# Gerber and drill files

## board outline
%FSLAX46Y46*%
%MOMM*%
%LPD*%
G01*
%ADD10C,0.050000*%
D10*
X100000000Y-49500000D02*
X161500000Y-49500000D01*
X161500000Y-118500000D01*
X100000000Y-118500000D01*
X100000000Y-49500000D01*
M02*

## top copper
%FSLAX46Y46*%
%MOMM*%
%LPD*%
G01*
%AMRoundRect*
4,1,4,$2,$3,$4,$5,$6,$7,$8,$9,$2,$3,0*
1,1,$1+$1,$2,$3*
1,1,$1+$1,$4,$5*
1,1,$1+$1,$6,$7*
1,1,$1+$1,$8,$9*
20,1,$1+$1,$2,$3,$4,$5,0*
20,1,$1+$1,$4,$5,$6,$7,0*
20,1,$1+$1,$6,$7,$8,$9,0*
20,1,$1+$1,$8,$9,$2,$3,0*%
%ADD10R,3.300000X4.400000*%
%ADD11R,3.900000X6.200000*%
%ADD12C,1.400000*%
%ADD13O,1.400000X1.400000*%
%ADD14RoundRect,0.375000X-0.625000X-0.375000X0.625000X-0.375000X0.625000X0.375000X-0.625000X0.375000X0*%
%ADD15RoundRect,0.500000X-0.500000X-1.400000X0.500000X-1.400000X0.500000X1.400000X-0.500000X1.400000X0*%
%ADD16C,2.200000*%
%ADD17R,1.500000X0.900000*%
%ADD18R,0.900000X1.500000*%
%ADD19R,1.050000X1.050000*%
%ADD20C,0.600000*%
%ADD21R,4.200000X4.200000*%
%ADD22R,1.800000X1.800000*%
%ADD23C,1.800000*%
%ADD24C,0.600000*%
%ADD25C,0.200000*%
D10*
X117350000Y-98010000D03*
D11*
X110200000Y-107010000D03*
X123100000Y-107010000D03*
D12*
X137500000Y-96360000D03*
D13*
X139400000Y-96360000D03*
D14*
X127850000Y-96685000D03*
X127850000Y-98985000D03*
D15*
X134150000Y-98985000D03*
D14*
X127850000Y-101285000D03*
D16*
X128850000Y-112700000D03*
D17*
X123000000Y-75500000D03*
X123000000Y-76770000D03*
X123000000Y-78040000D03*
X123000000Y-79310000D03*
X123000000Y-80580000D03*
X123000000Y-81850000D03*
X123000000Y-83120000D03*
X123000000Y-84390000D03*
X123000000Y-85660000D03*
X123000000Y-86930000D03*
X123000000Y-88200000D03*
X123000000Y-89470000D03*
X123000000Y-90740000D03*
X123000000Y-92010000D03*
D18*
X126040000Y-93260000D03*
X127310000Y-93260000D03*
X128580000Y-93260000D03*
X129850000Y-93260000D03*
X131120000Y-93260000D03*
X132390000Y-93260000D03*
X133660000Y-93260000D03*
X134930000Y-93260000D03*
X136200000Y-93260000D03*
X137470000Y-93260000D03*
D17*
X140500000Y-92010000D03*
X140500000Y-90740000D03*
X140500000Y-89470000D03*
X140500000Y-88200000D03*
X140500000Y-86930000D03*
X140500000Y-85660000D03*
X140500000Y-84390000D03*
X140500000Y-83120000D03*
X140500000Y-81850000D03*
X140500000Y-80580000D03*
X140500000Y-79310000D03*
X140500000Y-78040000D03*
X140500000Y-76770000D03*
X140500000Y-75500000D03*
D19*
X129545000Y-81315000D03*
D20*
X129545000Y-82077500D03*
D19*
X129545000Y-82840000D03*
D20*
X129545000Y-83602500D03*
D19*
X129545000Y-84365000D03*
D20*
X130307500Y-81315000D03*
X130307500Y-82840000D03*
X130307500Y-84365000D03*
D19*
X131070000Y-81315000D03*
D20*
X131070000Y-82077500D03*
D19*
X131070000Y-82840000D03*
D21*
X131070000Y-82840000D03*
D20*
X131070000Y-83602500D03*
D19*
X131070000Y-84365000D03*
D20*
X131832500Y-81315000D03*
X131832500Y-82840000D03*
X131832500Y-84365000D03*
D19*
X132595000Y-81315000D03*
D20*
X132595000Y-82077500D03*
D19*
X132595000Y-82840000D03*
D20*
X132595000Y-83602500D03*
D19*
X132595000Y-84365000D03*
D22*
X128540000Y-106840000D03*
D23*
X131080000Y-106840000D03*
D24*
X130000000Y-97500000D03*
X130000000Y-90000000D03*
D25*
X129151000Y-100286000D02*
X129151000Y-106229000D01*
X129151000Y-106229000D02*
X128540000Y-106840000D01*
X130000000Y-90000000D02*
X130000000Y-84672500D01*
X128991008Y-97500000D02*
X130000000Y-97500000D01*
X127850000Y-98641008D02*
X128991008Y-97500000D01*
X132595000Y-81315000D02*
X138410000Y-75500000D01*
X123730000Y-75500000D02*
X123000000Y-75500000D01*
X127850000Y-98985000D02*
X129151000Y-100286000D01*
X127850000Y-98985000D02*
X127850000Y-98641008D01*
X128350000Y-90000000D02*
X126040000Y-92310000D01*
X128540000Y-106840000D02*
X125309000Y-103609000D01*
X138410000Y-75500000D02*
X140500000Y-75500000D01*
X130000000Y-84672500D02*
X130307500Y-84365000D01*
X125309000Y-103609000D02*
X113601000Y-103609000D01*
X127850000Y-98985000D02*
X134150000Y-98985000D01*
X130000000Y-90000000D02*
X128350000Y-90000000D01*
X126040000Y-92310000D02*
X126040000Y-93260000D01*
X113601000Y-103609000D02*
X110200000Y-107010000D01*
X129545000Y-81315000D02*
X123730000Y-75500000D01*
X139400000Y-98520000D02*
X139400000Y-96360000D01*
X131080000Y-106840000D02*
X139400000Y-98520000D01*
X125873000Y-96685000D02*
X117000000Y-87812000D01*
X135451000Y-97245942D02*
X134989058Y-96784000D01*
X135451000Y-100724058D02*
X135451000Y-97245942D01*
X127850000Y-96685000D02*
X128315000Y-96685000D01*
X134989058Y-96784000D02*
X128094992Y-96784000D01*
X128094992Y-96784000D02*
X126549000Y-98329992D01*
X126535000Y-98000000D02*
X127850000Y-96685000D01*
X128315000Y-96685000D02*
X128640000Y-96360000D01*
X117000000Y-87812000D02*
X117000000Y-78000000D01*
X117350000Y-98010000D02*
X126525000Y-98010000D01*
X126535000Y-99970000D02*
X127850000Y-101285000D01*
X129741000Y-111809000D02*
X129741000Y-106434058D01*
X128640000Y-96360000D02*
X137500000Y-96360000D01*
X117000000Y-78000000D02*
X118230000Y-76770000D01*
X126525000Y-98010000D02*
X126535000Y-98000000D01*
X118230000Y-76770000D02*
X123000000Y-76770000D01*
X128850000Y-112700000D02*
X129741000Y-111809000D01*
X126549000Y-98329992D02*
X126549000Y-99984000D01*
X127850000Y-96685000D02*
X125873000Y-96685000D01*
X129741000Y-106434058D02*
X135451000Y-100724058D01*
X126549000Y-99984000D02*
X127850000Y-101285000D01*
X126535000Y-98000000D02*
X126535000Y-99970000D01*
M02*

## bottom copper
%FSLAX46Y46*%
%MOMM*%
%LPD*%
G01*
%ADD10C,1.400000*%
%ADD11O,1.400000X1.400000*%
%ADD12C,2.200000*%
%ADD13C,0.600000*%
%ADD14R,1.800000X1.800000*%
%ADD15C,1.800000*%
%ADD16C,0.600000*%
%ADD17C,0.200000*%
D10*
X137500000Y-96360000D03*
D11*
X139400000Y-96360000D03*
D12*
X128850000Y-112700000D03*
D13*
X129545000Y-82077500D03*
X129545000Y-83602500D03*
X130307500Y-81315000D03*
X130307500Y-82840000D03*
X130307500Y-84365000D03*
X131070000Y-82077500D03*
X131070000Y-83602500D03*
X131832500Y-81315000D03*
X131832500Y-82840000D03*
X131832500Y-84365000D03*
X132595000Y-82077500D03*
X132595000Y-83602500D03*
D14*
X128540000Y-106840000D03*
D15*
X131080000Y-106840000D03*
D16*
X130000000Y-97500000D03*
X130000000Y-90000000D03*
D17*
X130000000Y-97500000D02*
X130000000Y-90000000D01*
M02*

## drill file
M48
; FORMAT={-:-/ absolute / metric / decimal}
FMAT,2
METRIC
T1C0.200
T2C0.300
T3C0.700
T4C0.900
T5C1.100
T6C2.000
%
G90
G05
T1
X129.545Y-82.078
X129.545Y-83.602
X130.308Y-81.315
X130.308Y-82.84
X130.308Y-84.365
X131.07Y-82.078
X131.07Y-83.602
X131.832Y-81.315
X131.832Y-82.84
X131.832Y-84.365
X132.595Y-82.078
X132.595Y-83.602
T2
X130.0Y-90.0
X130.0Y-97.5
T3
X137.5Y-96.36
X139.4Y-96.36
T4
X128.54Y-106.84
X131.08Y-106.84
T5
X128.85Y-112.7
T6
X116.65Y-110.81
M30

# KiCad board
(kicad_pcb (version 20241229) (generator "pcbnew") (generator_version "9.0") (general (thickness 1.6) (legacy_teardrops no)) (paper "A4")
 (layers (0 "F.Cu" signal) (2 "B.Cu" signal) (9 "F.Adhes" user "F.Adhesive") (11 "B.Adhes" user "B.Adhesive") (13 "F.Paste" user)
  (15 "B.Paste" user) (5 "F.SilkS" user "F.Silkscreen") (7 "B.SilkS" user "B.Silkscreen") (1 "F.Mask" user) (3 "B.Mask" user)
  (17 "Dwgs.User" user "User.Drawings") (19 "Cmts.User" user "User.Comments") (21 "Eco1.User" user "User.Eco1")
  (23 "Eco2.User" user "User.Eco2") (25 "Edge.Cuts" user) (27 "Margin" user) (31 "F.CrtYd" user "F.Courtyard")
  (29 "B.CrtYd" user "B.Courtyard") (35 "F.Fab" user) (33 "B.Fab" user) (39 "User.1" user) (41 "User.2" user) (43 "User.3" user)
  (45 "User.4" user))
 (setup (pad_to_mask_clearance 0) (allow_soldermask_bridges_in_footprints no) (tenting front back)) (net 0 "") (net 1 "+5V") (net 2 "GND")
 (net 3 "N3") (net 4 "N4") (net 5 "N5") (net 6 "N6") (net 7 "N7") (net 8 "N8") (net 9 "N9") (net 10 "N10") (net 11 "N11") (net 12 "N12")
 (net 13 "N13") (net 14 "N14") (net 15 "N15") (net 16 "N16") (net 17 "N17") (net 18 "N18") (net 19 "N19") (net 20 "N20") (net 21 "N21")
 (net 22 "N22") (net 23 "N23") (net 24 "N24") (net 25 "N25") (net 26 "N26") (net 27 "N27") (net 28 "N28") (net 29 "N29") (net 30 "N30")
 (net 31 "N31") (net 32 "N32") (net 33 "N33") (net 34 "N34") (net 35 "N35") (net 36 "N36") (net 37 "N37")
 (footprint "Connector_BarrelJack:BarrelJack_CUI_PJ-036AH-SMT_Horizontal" (layer "F.Cu") (at 116.65 103.81)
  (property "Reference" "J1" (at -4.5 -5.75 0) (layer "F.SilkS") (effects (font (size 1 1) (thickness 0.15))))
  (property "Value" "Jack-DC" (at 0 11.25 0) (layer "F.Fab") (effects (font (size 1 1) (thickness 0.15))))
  (pad "" np_thru_hole circle (at 0 7) (size 2 2) (drill 2) (layers "*.Cu" "*.Mask"))
  (pad "1" smd rect (at 0.7 -5.8) (size 3.3 4.4) (layers "F.Cu" "F.Mask" "F.Paste") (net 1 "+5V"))
  (pad "2" smd rect (at -6.45 3.2) (size 3.9 6.2) (layers "F.Cu" "F.Mask" "F.Paste") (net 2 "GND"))
  (pad "3" smd rect (at 6.45 3.2) (size 3.9 6.2) (layers "F.Cu" "F.Mask" "F.Paste")))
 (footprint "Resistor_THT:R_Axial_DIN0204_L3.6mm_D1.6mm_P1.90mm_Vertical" (layer "F.Cu") (at 137.5 96.36)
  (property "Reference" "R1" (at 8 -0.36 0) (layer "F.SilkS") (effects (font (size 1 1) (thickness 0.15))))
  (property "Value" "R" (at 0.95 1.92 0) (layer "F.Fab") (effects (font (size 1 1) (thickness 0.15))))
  (pad "1" thru_hole circle (at 0 0) (size 1.4 1.4) (drill 0.7) (layers "*.Cu" "*.Mask") (remove_unused_layers no) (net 1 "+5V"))
  (pad "2" thru_hole oval (at 1.9 0) (size 1.4 1.4) (drill 0.7) (layers "*.Cu" "*.Mask") (remove_unused_layers no) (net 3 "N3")))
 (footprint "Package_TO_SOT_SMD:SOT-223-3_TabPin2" (layer "F.Cu") (at 131 98.985)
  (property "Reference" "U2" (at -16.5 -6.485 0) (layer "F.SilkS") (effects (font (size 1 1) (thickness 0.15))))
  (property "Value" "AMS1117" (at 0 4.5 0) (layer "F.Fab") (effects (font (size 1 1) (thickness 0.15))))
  (pad "1" smd roundrect (at -3.15 -2.3) (size 2 1.5) (layers "F.Cu" "F.Mask" "F.Paste") (roundrect_rratio 0.25) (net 1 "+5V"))
  (pad "2" smd roundrect (at -3.15 0) (size 2 1.5) (layers "F.Cu" "F.Mask" "F.Paste") (roundrect_rratio 0.25) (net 2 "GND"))
  (pad "2" smd roundrect (at 3.15 0) (size 2 3.8) (layers "F.Cu" "F.Mask" "F.Paste") (roundrect_rratio 0.25) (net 2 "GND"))
  (pad "3" smd roundrect (at -3.15 2.3) (size 2 1.5) (layers "F.Cu" "F.Mask" "F.Paste") (roundrect_rratio 0.25) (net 1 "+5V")))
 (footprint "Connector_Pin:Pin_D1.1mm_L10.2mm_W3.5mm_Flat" (layer "F.Cu") (at 128.85 112.7)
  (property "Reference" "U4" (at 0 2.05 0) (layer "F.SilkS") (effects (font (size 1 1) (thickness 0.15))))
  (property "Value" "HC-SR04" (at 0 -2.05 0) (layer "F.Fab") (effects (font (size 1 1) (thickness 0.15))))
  (pad "1" thru_hole circle (at 0 0) (size 2.2 2.2) (drill 1.1) (layers "*.Cu" "*.Mask") (remove_unused_layers no) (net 1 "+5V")))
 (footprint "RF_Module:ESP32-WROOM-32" (layer "F.Cu") (at 131.75 83.75)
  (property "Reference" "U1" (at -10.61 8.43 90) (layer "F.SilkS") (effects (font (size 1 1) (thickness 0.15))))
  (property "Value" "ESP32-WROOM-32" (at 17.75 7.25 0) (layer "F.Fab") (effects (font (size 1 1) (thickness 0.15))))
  (pad "1" smd rect (at -8.75 -8.25) (size 1.5 0.9) (layers "F.Cu" "F.Mask" "F.Paste") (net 2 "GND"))
  (pad "2" smd rect (at -8.75 -6.98) (size 1.5 0.9) (layers "F.Cu" "F.Mask" "F.Paste") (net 1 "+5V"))
  (pad "3" smd rect (at -8.75 -5.71) (size 1.5 0.9) (layers "F.Cu" "F.Mask" "F.Paste") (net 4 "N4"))
  (pad "4" smd rect (at -8.75 -4.44) (size 1.5 0.9) (layers "F.Cu" "F.Mask" "F.Paste") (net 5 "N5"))
  (pad "5" smd rect (at -8.75 -3.17) (size 1.5 0.9) (layers "F.Cu" "F.Mask" "F.Paste") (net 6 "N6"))
  (pad "6" smd rect (at -8.75 -1.9) (size 1.5 0.9) (layers "F.Cu" "F.Mask" "F.Paste") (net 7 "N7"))
  (pad "7" smd rect (at -8.75 -0.63) (size 1.5 0.9) (layers "F.Cu" "F.Mask" "F.Paste") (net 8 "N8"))
  (pad "8" smd rect (at -8.75 0.64) (size 1.5 0.9) (layers "F.Cu" "F.Mask" "F.Paste") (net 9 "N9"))
  (pad "9" smd rect (at -8.75 1.91) (size 1.5 0.9) (layers "F.Cu" "F.Mask" "F.Paste") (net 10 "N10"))
  (pad "10" smd rect (at -8.75 3.18) (size 1.5 0.9) (layers "F.Cu" "F.Mask" "F.Paste") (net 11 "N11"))
  (pad "11" smd rect (at -8.75 4.45) (size 1.5 0.9) (layers "F.Cu" "F.Mask" "F.Paste") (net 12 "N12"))
  (pad "12" smd rect (at -8.75 5.72) (size 1.5 0.9) (layers "F.Cu" "F.Mask" "F.Paste") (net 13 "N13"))
  (pad "13" smd rect (at -8.75 6.99) (size 1.5 0.9) (layers "F.Cu" "F.Mask" "F.Paste") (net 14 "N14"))
  (pad "14" smd rect (at -8.75 8.26) (size 1.5 0.9) (layers "F.Cu" "F.Mask" "F.Paste") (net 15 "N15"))
  (pad "15" smd rect (at -5.71 9.51 90) (size 1.5 0.9) (layers "F.Cu" "F.Mask" "F.Paste") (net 2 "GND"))
  (pad "16" smd rect (at -4.44 9.51 90) (size 1.5 0.9) (layers "F.Cu" "F.Mask" "F.Paste") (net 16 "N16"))
  (pad "17" smd rect (at -3.17 9.51 90) (size 1.5 0.9) (layers "F.Cu" "F.Mask" "F.Paste") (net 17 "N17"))
  (pad "18" smd rect (at -1.9 9.51 90) (size 1.5 0.9) (layers "F.Cu" "F.Mask" "F.Paste") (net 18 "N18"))
  (pad "19" smd rect (at -0.63 9.51 90) (size 1.5 0.9) (layers "F.Cu" "F.Mask" "F.Paste") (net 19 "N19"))
  (pad "20" smd rect (at 0.64 9.51 90) (size 1.5 0.9) (layers "F.Cu" "F.Mask" "F.Paste") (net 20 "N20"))
  (pad "21" smd rect (at 1.91 9.51 90) (size 1.5 0.9) (layers "F.Cu" "F.Mask" "F.Paste") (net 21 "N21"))
  (pad "22" smd rect (at 3.18 9.51 90) (size 1.5 0.9) (layers "F.Cu" "F.Mask" "F.Paste") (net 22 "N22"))
  (pad "23" smd rect (at 4.45 9.51 90) (size 1.5 0.9) (layers "F.Cu" "F.Mask" "F.Paste") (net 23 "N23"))
  (pad "24" smd rect (at 5.72 9.51 90) (size 1.5 0.9) (layers "F.Cu" "F.Mask" "F.Paste") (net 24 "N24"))
  (pad "25" smd rect (at 8.75 8.26) (size 1.5 0.9) (layers "F.Cu" "F.Mask" "F.Paste") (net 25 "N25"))
  (pad "26" smd rect (at 8.75 6.99) (size 1.5 0.9) (layers "F.Cu" "F.Mask" "F.Paste") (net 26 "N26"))
  (pad "27" smd rect (at 8.75 5.72) (size 1.5 0.9) (layers "F.Cu" "F.Mask" "F.Paste") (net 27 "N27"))
  (pad "28" smd rect (at 8.75 4.45) (size 1.5 0.9) (layers "F.Cu" "F.Mask" "F.Paste") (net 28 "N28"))
  (pad "29" smd rect (at 8.75 3.18) (size 1.5 0.9) (layers "F.Cu" "F.Mask" "F.Paste") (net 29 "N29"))
  (pad "30" smd rect (at 8.75 1.91) (size 1.5 0.9) (layers "F.Cu" "F.Mask" "F.Paste") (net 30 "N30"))
  (pad "31" smd rect (at 8.75 0.64) (size 1.5 0.9) (layers "F.Cu" "F.Mask" "F.Paste") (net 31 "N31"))
  (pad "32" smd rect (at 8.75 -0.63) (size 1.5 0.9) (layers "F.Cu" "F.Mask" "F.Paste") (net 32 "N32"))
  (pad "33" smd rect (at 8.75 -1.9) (size 1.5 0.9) (layers "F.Cu" "F.Mask" "F.Paste") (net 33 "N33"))
  (pad "34" smd rect (at 8.75 -3.17) (size 1.5 0.9) (layers "F.Cu" "F.Mask" "F.Paste") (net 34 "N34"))
  (pad "35" smd rect (at 8.75 -4.44) (size 1.5 0.9) (layers "F.Cu" "F.Mask" "F.Paste") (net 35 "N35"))
  (pad "36" smd rect (at 8.75 -5.71) (size 1.5 0.9) (layers "F.Cu" "F.Mask" "F.Paste") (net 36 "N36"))
  (pad "37" smd rect (at 8.75 -6.98) (size 1.5 0.9) (layers "F.Cu" "F.Mask" "F.Paste") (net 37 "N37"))
  (pad "38" smd rect (at 8.75 -8.25) (size 1.5 0.9) (layers "F.Cu" "F.Mask" "F.Paste") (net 2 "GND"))
  (pad "39" smd rect (at -2.205 -2.435) (size 1.05 1.05) (layers "F.Cu" "F.Paste") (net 2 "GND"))
  (pad "39" thru_hole circle (at -2.205 -1.6725) (size 0.6 0.6) (drill 0.2) (layers "*.Cu" "F.Mask") (remove_unused_layers no) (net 2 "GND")
   (zone_connect 2))
  (pad "39" smd rect (at -2.205 -0.91) (size 1.05 1.05) (layers "F.Cu" "F.Paste") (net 2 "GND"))
  (pad "39" thru_hole circle (at -2.205 -0.1475) (size 0.6 0.6) (drill 0.2) (layers "*.Cu" "F.Mask") (remove_unused_layers no) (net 2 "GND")
   (zone_connect 2))
  (pad "39" smd rect (at -2.205 0.615) (size 1.05 1.05) (layers "F.Cu" "F.Paste") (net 2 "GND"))
  (pad "39" thru_hole circle (at -1.4425 -2.435) (size 0.6 0.6) (drill 0.2) (layers "*.Cu" "F.Mask") (remove_unused_layers no) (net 2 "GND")
   (zone_connect 2))
  (pad "39" thru_hole circle (at -1.4425 -0.91) (size 0.6 0.6) (drill 0.2) (layers "*.Cu" "F.Mask") (remove_unused_layers no) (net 2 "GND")
   (zone_connect 2))
  (pad "39" thru_hole circle (at -1.4425 0.615) (size 0.6 0.6) (drill 0.2) (layers "*.Cu" "F.Mask") (remove_unused_layers no) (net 2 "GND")
   (zone_connect 2))
  (pad "39" smd rect (at -0.68 -2.435) (size 1.05 1.05) (layers "F.Cu" "F.Paste") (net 2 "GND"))
  (pad "39" thru_hole circle (at -0.68 -1.6725) (size 0.6 0.6) (drill 0.2) (layers "*.Cu" "F.Mask") (remove_unused_layers no) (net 2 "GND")
   (zone_connect 2))
  (pad "39" smd rect (at -0.68 -0.91) (size 1.05 1.05) (layers "F.Cu" "F.Paste") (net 2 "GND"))
  (pad "39" smd rect (at -0.68 -0.91) (size 4.2 4.2) (layers "F.Cu" "F.Mask") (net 2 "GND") (zone_connect 2))
  (pad "39" thru_hole circle (at -0.68 -0.1475) (size 0.6 0.6) (drill 0.2) (layers "*.Cu" "F.Mask") (remove_unused_layers no) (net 2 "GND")
   (zone_connect 2))
  (pad "39" smd rect (at -0.68 0.615) (size 1.05 1.05) (layers "F.Cu" "F.Paste") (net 2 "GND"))
  (pad "39" thru_hole circle (at 0.0825 -2.435) (size 0.6 0.6) (drill 0.2) (layers "*.Cu" "F.Mask") (remove_unused_layers no) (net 2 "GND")
   (zone_connect 2))
  (pad "39" thru_hole circle (at 0.0825 -0.91) (size 0.6 0.6) (drill 0.2) (layers "*.Cu" "F.Mask") (remove_unused_layers no) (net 2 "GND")
   (zone_connect 2))
  (pad "39" thru_hole circle (at 0.0825 0.615) (size 0.6 0.6) (drill 0.2) (layers "*.Cu" "F.Mask") (remove_unused_layers no) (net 2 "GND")
   (zone_connect 2))
  (pad "39" smd rect (at 0.845 -2.435) (size 1.05 1.05) (layers "F.Cu" "F.Paste") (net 2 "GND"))
  (pad "39" thru_hole circle (at 0.845 -1.6725) (size 0.6 0.6) (drill 0.2) (layers "*.Cu" "F.Mask") (remove_unused_layers no) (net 2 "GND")
   (zone_connect 2))
  (pad "39" smd rect (at 0.845 -0.91) (size 1.05 1.05) (layers "F.Cu" "F.Paste") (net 2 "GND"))
  (pad "39" thru_hole circle (at 0.845 -0.1475) (size 0.6 0.6) (drill 0.2) (layers "*.Cu" "F.Mask") (remove_unused_layers no) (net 2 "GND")
   (zone_connect 2))
  (pad "39" smd rect (at 0.845 0.615) (size 1.05 1.05) (layers "F.Cu" "F.Paste") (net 2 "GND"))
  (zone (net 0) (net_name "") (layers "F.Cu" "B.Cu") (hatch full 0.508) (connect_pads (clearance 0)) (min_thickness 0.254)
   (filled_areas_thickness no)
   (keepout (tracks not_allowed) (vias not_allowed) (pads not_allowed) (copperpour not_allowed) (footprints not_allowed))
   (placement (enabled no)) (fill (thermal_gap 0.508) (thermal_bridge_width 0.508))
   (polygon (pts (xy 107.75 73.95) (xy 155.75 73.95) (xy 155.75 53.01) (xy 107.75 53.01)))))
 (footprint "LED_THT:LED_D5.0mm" (layer "F.Cu") (at 128.54 106.84)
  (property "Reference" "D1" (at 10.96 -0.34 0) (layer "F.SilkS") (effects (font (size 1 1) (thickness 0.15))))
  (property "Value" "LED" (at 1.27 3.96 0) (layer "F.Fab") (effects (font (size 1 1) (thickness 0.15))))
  (pad "1" thru_hole rect (at 0 0) (size 1.8 1.8) (drill 0.9) (layers "*.Cu" "*.Mask") (remove_unused_layers no) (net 2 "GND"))
  (pad "2" thru_hole circle (at 2.54 0) (size 1.8 1.8) (drill 0.9) (layers "*.Cu" "*.Mask") (remove_unused_layers no) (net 3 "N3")))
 (gr_rect (start 100 49.5) (end 161.5 118.5) (stroke (width 0.05) (type default)) (fill no) (layer "Edge.Cuts"))
 (segment (start 129.151 100.286) (end 129.151 106.229) (width 0.2) (layer "F.Cu") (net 2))
 (segment (start 129.151 106.229) (end 128.54 106.84) (width 0.2) (layer "F.Cu") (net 2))
 (segment (start 130 90) (end 130 84.6725) (width 0.2) (layer "F.Cu") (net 2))
 (segment (start 128.991008 97.5) (end 130 97.5) (width 0.2) (layer "F.Cu") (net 2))
 (segment (start 127.85 98.641008) (end 128.991008 97.5) (width 0.2) (layer "F.Cu") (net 2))
 (segment (start 132.595 81.315) (end 138.41 75.5) (width 0.2) (layer "F.Cu") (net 2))
 (segment (start 123.73 75.5) (end 123 75.5) (width 0.2) (layer "F.Cu") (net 2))
 (segment (start 127.85 98.985) (end 129.151 100.286) (width 0.2) (layer "F.Cu") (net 2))
 (segment (start 127.85 98.985) (end 127.85 98.641008) (width 0.2) (layer "F.Cu") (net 2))
 (segment (start 128.35 90) (end 126.04 92.31) (width 0.2) (layer "F.Cu") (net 2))
 (segment (start 128.54 106.84) (end 125.309 103.609) (width 0.2) (layer "F.Cu") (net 2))
 (segment (start 138.41 75.5) (end 140.5 75.5) (width 0.2) (layer "F.Cu") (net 2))
 (segment (start 130 84.6725) (end 130.3075 84.365) (width 0.2) (layer "F.Cu") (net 2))
 (segment (start 125.309 103.609) (end 113.601 103.609) (width 0.2) (layer "F.Cu") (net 2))
 (segment (start 127.85 98.985) (end 134.15 98.985) (width 0.2) (layer "F.Cu") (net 2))
 (segment (start 130 90) (end 128.35 90) (width 0.2) (layer "F.Cu") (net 2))
 (segment (start 126.04 92.31) (end 126.04 93.26) (width 0.2) (layer "F.Cu") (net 2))
 (segment (start 113.601 103.609) (end 110.2 107.01) (width 0.2) (layer "F.Cu") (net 2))
 (segment (start 129.545 81.315) (end 123.73 75.5) (width 0.2) (layer "F.Cu") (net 2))
 (via (at 130 97.5) (size 0.6) (drill 0.3) (layers "F.Cu" "B.Cu") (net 2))
 (via (at 130 90) (size 0.6) (drill 0.3) (layers "F.Cu" "B.Cu") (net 2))
 (segment (start 130 97.5) (end 130 90) (width 0.2) (layer "B.Cu") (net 2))
 (segment (start 139.4 98.52) (end 139.4 96.36) (width 0.2) (layer "F.Cu") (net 3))
 (segment (start 131.08 106.84) (end 139.4 98.52) (width 0.2) (layer "F.Cu") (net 3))
 (segment (start 125.873 96.685) (end 117 87.812) (width 0.2) (layer "F.Cu") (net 1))
 (segment (start 135.451 97.245942) (end 134.989058 96.784) (width 0.2) (layer "F.Cu") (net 1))
 (segment (start 135.451 100.724058) (end 135.451 97.245942) (width 0.2) (layer "F.Cu") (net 1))
 (segment (start 127.85 96.685) (end 128.315 96.685) (width 0.2) (layer "F.Cu") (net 1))
 (segment (start 134.989058 96.784) (end 128.094992 96.784) (width 0.2) (layer "F.Cu") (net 1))
 (segment (start 128.094992 96.784) (end 126.549 98.329992) (width 0.2) (layer "F.Cu") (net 1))
 (segment (start 126.535 98) (end 127.85 96.685) (width 0.2) (layer "F.Cu") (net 1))
 (segment (start 128.315 96.685) (end 128.64 96.36) (width 0.2) (layer "F.Cu") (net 1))
 (segment (start 117 87.812) (end 117 78) (width 0.2) (layer "F.Cu") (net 1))
 (segment (start 117.35 98.01) (end 126.525 98.01) (width 0.2) (layer "F.Cu") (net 1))
 (segment (start 126.535 99.97) (end 127.85 101.285) (width 0.2) (layer "F.Cu") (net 1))
 (segment (start 129.741 111.809) (end 129.741 106.434058) (width 0.2) (layer "F.Cu") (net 1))
 (segment (start 128.64 96.36) (end 137.5 96.36) (width 0.2) (layer "F.Cu") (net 1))
 (segment (start 117 78) (end 118.23 76.77) (width 0.2) (layer "F.Cu") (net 1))
 (segment (start 126.525 98.01) (end 126.535 98) (width 0.2) (layer "F.Cu") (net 1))
 (segment (start 118.23 76.77) (end 123 76.77) (width 0.2) (layer "F.Cu") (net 1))
 (segment (start 128.85 112.7) (end 129.741 111.809) (width 0.2) (layer "F.Cu") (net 1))
 (segment (start 126.549 98.329992) (end 126.549 99.984) (width 0.2) (layer "F.Cu") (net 1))
 (segment (start 127.85 96.685) (end 125.873 96.685) (width 0.2) (layer "F.Cu") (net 1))
 (segment (start 129.741 106.434058) (end 135.451 100.724058) (width 0.2) (layer "F.Cu") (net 1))
 (segment (start 126.549 99.984) (end 127.85 101.285) (width 0.2) (layer "F.Cu") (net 1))
 (segment (start 126.535 98) (end 126.535 99.97) (width 0.2) (layer "F.Cu") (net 1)))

